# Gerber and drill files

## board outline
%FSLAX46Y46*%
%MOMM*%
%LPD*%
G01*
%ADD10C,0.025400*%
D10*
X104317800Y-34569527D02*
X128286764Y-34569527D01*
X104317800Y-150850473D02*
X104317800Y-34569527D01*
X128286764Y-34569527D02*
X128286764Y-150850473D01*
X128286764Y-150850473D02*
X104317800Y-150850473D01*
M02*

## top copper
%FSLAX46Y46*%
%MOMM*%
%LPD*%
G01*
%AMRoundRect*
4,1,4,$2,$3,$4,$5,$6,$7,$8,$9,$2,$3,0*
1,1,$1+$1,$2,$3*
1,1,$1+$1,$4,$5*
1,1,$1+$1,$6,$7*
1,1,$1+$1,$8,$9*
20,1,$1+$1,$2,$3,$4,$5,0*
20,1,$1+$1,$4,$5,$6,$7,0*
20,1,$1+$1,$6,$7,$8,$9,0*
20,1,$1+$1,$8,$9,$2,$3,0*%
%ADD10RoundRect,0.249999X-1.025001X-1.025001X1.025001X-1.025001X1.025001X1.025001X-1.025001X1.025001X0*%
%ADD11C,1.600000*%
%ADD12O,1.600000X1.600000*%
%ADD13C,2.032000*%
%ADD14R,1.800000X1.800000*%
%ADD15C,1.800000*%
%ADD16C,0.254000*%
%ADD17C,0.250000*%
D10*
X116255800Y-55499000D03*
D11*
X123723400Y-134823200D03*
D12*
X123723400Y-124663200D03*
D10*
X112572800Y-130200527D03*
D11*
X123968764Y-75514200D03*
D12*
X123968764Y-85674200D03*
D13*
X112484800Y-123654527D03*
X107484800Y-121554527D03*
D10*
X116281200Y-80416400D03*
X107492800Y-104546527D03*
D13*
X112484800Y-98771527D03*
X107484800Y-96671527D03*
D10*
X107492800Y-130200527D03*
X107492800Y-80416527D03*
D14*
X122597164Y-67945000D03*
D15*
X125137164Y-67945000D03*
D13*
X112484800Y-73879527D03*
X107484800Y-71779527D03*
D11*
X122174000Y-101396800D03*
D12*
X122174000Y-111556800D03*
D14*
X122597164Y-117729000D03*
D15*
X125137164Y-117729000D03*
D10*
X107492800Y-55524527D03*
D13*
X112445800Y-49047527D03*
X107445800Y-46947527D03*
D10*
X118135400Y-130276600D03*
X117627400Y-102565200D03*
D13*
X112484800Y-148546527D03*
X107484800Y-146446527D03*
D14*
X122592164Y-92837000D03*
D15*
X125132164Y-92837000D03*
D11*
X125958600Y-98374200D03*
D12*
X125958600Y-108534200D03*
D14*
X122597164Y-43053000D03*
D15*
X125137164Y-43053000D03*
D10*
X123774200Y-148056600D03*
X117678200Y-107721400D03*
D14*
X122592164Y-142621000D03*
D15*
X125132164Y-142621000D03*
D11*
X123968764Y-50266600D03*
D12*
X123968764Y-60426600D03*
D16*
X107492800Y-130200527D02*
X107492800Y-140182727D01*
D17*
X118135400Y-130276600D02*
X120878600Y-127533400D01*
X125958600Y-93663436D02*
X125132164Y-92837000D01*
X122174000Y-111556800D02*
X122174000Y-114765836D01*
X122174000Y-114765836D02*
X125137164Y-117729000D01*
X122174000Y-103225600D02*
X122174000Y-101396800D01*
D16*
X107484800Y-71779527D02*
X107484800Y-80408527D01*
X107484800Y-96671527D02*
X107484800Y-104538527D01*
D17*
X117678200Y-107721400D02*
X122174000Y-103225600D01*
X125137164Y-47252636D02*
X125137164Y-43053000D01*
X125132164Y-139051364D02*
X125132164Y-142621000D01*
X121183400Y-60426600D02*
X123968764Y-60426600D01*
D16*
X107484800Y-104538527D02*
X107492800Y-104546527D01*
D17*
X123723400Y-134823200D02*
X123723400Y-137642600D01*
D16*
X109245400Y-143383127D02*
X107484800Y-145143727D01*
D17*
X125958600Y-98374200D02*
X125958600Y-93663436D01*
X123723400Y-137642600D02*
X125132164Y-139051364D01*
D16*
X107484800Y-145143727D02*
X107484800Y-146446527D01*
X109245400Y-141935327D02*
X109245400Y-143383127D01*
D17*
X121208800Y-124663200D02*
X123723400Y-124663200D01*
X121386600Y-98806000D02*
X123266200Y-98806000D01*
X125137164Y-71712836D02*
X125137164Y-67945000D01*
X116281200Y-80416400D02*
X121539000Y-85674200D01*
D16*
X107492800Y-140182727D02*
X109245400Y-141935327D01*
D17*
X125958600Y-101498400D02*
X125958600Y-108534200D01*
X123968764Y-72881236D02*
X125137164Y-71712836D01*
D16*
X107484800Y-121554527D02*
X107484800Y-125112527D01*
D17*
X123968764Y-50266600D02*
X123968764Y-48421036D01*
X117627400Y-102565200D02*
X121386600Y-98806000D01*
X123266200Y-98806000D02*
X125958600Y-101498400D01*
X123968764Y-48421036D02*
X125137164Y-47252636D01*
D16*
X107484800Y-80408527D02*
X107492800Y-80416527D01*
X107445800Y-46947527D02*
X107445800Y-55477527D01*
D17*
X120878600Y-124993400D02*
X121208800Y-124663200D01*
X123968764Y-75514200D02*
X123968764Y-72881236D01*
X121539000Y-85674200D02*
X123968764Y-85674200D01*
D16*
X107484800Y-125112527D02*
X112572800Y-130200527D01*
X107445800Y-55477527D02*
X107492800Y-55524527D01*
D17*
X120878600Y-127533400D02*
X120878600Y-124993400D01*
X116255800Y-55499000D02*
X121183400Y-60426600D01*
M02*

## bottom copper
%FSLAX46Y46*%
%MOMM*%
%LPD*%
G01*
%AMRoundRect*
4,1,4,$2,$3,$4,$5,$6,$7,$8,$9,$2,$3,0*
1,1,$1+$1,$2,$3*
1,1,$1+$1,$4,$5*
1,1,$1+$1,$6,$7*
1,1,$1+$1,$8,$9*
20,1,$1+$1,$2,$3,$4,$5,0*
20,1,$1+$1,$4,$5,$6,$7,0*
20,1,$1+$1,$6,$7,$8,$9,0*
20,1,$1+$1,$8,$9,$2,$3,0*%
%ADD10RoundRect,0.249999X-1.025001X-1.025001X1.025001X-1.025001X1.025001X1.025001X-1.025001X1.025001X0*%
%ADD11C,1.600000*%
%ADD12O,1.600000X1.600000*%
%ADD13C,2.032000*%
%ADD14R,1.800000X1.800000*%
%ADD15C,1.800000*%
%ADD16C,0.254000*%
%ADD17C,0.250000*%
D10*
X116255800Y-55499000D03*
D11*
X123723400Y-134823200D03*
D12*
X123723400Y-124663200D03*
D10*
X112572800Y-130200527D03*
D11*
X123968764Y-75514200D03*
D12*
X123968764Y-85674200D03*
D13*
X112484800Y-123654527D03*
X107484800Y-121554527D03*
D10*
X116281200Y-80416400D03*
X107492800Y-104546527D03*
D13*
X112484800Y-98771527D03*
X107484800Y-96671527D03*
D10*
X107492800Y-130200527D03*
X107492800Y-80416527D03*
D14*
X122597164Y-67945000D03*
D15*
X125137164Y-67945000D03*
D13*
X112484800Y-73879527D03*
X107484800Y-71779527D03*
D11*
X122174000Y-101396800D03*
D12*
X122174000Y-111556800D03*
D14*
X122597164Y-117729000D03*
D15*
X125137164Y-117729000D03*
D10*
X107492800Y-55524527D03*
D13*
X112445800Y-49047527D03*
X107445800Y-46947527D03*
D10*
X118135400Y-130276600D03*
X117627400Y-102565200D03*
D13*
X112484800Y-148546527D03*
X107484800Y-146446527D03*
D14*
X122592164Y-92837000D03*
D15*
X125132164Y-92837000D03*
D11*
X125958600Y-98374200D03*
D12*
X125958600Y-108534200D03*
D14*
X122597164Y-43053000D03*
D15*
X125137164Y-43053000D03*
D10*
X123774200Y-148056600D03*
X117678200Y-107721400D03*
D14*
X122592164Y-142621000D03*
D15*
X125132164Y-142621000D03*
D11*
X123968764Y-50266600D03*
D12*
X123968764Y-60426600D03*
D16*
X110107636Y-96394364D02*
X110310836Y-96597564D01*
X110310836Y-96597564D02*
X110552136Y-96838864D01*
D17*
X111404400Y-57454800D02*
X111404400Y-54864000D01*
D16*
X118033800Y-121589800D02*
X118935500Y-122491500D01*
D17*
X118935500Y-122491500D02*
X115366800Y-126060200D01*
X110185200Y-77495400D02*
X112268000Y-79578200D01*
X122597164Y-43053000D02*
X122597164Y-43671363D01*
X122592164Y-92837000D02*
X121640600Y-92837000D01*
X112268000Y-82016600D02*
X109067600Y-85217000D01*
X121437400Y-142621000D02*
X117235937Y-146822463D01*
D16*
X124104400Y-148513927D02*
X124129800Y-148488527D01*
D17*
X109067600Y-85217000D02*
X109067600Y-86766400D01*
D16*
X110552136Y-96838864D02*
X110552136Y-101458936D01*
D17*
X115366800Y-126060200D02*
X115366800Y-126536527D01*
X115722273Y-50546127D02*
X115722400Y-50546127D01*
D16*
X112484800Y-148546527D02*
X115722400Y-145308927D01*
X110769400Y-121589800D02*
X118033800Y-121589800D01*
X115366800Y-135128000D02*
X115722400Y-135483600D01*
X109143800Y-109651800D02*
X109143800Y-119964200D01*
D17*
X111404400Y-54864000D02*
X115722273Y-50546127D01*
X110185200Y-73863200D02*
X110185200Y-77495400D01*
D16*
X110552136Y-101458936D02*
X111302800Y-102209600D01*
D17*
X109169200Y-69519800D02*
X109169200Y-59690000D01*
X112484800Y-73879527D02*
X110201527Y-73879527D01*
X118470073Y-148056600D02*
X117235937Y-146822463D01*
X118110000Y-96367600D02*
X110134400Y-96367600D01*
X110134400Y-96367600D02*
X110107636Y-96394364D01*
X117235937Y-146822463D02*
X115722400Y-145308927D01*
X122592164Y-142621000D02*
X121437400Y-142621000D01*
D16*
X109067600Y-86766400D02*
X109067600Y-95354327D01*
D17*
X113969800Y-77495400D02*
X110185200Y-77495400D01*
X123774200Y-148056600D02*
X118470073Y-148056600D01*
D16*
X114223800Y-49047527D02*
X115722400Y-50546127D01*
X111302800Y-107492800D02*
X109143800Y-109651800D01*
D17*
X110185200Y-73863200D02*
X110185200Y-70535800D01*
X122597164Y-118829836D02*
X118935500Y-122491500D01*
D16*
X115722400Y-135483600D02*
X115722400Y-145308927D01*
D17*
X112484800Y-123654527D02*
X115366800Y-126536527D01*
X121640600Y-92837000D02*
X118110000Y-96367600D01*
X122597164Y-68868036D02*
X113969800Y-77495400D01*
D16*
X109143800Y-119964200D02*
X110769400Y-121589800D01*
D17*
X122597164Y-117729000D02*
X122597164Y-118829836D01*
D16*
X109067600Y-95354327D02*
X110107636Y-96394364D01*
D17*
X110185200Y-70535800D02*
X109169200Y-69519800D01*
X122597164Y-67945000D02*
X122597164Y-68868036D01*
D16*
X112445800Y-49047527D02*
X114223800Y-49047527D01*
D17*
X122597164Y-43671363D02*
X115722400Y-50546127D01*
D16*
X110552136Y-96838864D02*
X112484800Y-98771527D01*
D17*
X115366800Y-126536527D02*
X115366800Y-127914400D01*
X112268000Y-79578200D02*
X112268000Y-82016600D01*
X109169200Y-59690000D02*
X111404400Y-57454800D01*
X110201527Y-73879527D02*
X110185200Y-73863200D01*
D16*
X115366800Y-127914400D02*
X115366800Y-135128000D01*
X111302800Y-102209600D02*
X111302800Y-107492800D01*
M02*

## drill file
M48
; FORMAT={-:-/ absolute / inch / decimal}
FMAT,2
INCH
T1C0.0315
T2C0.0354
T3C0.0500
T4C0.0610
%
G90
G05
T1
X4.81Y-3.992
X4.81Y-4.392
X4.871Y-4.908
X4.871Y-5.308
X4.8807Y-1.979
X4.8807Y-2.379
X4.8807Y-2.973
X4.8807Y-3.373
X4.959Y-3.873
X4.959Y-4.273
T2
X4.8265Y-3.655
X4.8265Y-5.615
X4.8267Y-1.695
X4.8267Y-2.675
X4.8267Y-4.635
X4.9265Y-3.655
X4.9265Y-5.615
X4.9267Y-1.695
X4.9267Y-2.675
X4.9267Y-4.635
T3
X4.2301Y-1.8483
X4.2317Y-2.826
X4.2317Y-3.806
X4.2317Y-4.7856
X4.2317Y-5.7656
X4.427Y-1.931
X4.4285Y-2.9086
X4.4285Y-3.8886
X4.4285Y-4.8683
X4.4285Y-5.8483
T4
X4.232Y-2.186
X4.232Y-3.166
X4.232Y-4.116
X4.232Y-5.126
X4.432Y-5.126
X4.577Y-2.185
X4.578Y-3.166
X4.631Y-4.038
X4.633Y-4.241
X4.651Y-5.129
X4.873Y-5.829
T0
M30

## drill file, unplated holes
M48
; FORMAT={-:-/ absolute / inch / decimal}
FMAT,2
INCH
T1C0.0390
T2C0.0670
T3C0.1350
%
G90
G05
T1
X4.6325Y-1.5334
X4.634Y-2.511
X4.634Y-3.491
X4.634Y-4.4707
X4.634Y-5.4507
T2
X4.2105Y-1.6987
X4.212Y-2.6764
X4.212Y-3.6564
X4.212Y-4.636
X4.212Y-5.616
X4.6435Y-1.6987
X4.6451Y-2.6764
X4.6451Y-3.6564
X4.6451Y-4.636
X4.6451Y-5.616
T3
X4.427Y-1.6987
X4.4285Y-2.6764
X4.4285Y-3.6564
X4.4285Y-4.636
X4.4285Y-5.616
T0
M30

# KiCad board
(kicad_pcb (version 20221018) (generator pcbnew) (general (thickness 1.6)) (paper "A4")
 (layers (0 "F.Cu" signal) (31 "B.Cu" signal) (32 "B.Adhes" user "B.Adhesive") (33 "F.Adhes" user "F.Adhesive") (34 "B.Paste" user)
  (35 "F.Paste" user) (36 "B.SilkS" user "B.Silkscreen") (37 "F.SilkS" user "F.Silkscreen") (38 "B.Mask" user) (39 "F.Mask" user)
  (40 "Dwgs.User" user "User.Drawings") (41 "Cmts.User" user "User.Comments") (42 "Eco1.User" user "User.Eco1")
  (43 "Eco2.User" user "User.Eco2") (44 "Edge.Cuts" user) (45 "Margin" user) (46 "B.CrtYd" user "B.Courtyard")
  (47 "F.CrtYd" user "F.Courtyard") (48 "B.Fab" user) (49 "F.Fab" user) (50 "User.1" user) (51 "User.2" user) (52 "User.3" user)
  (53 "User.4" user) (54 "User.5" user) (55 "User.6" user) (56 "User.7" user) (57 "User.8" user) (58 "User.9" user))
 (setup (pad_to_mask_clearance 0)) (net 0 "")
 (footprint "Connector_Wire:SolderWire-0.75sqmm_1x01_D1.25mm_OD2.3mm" (layer "F.Cu") (at 116.2558 55.499)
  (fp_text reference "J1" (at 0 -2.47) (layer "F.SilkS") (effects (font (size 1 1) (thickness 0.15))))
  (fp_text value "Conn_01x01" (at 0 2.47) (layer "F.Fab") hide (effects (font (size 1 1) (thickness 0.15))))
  (pad "1" thru_hole roundrect (at 0 0) (size 2.55 2.55) (drill 1.55) (layers "*.Cu" "*.Mask") (roundrect_rratio 0.09803882353)))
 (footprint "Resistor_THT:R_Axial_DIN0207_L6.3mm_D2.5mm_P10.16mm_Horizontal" (layer "F.Cu") (at 123.7234 134.8232 90)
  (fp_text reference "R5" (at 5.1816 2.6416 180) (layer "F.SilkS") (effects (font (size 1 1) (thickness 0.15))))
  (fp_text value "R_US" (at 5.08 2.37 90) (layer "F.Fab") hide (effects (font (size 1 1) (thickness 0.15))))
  (pad "1" thru_hole circle (at 0 0 90) (size 1.6 1.6) (drill 0.8) (layers "*.Cu" "*.Mask"))
  (pad "2" thru_hole oval (at 10.16 0 90) (size 1.6 1.6) (drill 0.8) (layers "*.Cu" "*.Mask")))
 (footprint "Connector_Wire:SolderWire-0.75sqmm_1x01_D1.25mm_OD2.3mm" (layer "F.Cu") (at 112.5728 130.200527)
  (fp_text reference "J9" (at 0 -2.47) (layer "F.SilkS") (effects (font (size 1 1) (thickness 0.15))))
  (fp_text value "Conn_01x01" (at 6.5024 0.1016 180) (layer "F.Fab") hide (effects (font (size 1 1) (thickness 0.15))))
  (pad "1" thru_hole roundrect (at 0 0) (size 2.55 2.55) (drill 1.55) (layers "*.Cu" "*.Mask") (roundrect_rratio 0.09803882353)))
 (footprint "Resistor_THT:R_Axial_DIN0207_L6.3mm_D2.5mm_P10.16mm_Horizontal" (layer "F.Cu") (at 123.968764 75.5142 -90)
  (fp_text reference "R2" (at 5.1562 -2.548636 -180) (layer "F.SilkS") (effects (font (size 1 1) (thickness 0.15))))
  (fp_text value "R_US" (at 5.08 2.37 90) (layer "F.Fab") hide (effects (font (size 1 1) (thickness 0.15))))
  (pad "1" thru_hole circle (at 0 0 270) (size 1.6 1.6) (drill 0.8) (layers "*.Cu" "*.Mask"))
  (pad "2" thru_hole oval (at 10.16 0 270) (size 1.6 1.6) (drill 0.8) (layers "*.Cu" "*.Mask")))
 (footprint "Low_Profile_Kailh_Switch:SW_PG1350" (layer "F.Cu") (at 112.4848 117.754527)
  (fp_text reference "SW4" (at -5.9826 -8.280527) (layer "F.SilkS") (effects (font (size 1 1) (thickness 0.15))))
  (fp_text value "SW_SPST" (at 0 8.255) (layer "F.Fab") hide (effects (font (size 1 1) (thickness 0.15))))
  (pad "" np_thru_hole circle (at -5.5 0) (size 1.7018 1.7018) (drill 1.7018) (layers "F&B.Cu" "*.Mask"))
  (pad "" np_thru_hole circle (at 0 0) (size 3.429 3.429) (drill 3.429) (layers "F&B.Cu" "*.Mask"))
  (pad "" np_thru_hole circle (at 5.22 -4.2) (size 0.9906 0.9906) (drill 0.9906) (layers "F&B.Cu" "*.Mask"))
  (pad "" np_thru_hole circle (at 5.5 0) (size 1.7018 1.7018) (drill 1.7018) (layers "F&B.Cu" "*.Mask"))
  (pad "1" thru_hole circle (at 0 5.9) (size 2.032 2.032) (drill 1.27) (layers "*.Cu" "*.Mask"))
  (pad "2" thru_hole circle (at -5 3.8) (size 2.032 2.032) (drill 1.27) (layers "*.Cu" "*.Mask")))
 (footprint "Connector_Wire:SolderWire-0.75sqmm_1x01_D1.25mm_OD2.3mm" (layer "F.Cu") (at 116.2812 80.4164)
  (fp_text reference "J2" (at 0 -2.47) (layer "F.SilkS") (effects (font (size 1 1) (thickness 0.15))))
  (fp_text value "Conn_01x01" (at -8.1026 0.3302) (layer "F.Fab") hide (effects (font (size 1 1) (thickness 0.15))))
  (pad "1" thru_hole roundrect (at 0 0) (size 2.55 2.55) (drill 1.55) (layers "*.Cu" "*.Mask") (roundrect_rratio 0.09803882353)))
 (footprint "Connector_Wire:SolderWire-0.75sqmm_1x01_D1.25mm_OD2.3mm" (layer "F.Cu") (at 107.4928 104.546527)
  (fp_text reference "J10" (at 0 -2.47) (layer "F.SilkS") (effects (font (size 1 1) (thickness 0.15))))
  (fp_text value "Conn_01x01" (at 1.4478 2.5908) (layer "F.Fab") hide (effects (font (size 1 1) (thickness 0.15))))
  (pad "1" thru_hole roundrect (at 0 0) (size 2.55 2.55) (drill 1.55) (layers "*.Cu" "*.Mask") (roundrect_rratio 0.09803882353)))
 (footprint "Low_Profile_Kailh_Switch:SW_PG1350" (layer "F.Cu") (at 112.4848 92.871527)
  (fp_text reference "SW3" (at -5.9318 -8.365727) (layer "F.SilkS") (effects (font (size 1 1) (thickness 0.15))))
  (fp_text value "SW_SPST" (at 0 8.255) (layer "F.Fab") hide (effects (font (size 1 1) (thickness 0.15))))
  (pad "" np_thru_hole circle (at -5.5 0) (size 1.7018 1.7018) (drill 1.7018) (layers "F&B.Cu" "*.Mask"))
  (pad "" np_thru_hole circle (at 0 0) (size 3.429 3.429) (drill 3.429) (layers "F&B.Cu" "*.Mask"))
  (pad "" np_thru_hole circle (at 5.22 -4.2) (size 0.9906 0.9906) (drill 0.9906) (layers "F&B.Cu" "*.Mask"))
  (pad "" np_thru_hole circle (at 5.5 0) (size 1.7018 1.7018) (drill 1.7018) (layers "F&B.Cu" "*.Mask"))
  (pad "1" thru_hole circle (at 0 5.9) (size 2.032 2.032) (drill 1.27) (layers "*.Cu" "*.Mask"))
  (pad "2" thru_hole circle (at -5 3.8) (size 2.032 2.032) (drill 1.27) (layers "*.Cu" "*.Mask")))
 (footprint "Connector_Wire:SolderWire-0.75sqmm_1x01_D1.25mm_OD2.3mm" (layer "F.Cu") (at 107.4928 130.200527)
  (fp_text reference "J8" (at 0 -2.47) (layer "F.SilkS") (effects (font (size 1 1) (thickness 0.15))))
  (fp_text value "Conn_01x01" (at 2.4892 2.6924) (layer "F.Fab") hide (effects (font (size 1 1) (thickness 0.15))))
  (pad "1" thru_hole roundrect (at 0 0) (size 2.55 2.55) (drill 1.55) (layers "*.Cu" "*.Mask") (roundrect_rratio 0.09803882353)))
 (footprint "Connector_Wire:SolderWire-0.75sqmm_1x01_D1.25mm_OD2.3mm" (layer "F.Cu") (at 107.4928 80.416527)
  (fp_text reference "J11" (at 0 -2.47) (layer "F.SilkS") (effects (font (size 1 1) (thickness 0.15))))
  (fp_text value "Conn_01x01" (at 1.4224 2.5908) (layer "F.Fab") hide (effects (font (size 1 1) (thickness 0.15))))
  (pad "1" thru_hole roundrect (at 0 0) (size 2.55 2.55) (drill 1.55) (layers "*.Cu" "*.Mask") (roundrect_rratio 0.09803882353)))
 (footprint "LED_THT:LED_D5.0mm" (layer "F.Cu") (at 122.597164 67.945)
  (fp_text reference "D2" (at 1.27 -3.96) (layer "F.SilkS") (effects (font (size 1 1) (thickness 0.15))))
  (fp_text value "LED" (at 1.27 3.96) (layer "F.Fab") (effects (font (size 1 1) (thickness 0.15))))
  (pad "1" thru_hole rect (at 0 0) (size 1.8 1.8) (drill 0.9) (layers "*.Cu" "*.Mask"))
  (pad "2" thru_hole circle (at 2.54 0) (size 1.8 1.8) (drill 0.9) (layers "*.Cu" "*.Mask")))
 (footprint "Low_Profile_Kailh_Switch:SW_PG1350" (layer "F.Cu") (at 112.4848 67.979527)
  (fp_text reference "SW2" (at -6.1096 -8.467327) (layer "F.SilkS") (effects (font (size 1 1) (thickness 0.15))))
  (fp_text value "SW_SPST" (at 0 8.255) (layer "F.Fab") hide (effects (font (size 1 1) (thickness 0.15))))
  (pad "" np_thru_hole circle (at -5.5 0) (size 1.7018 1.7018) (drill 1.7018) (layers "F&B.Cu" "*.Mask"))
  (pad "" np_thru_hole circle (at 0 0) (size 3.429 3.429) (drill 3.429) (layers "F&B.Cu" "*.Mask"))
  (pad "" np_thru_hole circle (at 5.22 -4.2) (size 0.9906 0.9906) (drill 0.9906) (layers "F&B.Cu" "*.Mask"))
  (pad "" np_thru_hole circle (at 5.5 0) (size 1.7018 1.7018) (drill 1.7018) (layers "F&B.Cu" "*.Mask"))
  (pad "1" thru_hole circle (at 0 5.9) (size 2.032 2.032) (drill 1.27) (layers "*.Cu" "*.Mask"))
  (pad "2" thru_hole circle (at -5 3.8) (size 2.032 2.032) (drill 1.27) (layers "*.Cu" "*.Mask")))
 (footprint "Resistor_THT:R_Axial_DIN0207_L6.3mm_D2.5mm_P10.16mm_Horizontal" (layer "F.Cu") (at 122.174 101.3968 -90)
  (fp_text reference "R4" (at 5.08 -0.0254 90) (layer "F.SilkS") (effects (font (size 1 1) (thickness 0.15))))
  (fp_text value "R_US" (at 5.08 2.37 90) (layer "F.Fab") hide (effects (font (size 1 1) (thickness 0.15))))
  (pad "1" thru_hole circle (at 0 0 270) (size 1.6 1.6) (drill 0.8) (layers "*.Cu" "*.Mask"))
  (pad "2" thru_hole oval (at 10.16 0 270) (size 1.6 1.6) (drill 0.8) (layers "*.Cu" "*.Mask")))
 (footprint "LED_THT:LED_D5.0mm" (layer "F.Cu") (at 122.597164 117.729)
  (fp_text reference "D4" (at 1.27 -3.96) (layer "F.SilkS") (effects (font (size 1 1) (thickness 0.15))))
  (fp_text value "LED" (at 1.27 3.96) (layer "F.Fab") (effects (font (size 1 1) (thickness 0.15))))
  (pad "1" thru_hole rect (at 0 0) (size 1.8 1.8) (drill 0.9) (layers "*.Cu" "*.Mask"))
  (pad "2" thru_hole circle (at 2.54 0) (size 1.8 1.8) (drill 0.9) (layers "*.Cu" "*.Mask")))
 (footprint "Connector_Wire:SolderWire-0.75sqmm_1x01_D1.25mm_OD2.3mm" (layer "F.Cu") (at 107.4928 55.524527)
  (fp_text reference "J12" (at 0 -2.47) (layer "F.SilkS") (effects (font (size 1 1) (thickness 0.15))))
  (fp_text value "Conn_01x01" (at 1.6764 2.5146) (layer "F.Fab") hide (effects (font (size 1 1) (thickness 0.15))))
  (pad "1" thru_hole roundrect (at 0 0) (size 2.55 2.55) (drill 1.55) (layers "*.Cu" "*.Mask") (roundrect_rratio 0.09803882353)))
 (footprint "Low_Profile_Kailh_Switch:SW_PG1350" (layer "F.Cu") (at 112.4458 43.147527)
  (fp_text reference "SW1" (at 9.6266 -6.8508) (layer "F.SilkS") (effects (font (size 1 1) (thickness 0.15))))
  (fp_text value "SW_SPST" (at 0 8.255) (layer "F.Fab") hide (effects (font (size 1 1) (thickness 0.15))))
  (pad "" np_thru_hole circle (at -5.5 0) (size 1.7018 1.7018) (drill 1.7018) (layers "F&B.Cu" "*.Mask"))
  (pad "" np_thru_hole circle (at 0 0) (size 3.429 3.429) (drill 3.429) (layers "F&B.Cu" "*.Mask"))
  (pad "" np_thru_hole circle (at 5.22 -4.2) (size 0.9906 0.9906) (drill 0.9906) (layers "F&B.Cu" "*.Mask"))
  (pad "" np_thru_hole circle (at 5.5 0) (size 1.7018 1.7018) (drill 1.7018) (layers "F&B.Cu" "*.Mask"))
  (pad "1" thru_hole circle (at 0 5.9) (size 2.032 2.032) (drill 1.27) (layers "*.Cu" "*.Mask"))
  (pad "2" thru_hole circle (at -5 3.8) (size 2.032 2.032) (drill 1.27) (layers "*.Cu" "*.Mask")))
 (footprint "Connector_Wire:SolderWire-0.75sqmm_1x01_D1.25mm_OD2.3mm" (layer "F.Cu") (at 118.1354 130.2766)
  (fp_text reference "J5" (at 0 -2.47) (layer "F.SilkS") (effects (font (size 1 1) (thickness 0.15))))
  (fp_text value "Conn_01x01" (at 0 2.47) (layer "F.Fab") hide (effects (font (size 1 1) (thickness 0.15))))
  (pad "1" thru_hole roundrect (at 0 0) (size 2.55 2.55) (drill 1.55) (layers "*.Cu" "*.Mask") (roundrect_rratio 0.09803882353)))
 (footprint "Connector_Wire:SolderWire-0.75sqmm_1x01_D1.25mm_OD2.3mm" (layer "F.Cu") (at 117.6274 102.5652)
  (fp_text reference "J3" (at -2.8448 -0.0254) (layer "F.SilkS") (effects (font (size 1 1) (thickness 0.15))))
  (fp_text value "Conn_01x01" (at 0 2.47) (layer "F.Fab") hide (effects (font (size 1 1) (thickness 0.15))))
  (pad "1" thru_hole roundrect (at 0 0) (size 2.55 2.55) (drill 1.55) (layers "*.Cu" "*.Mask") (roundrect_rratio 0.09803882353)))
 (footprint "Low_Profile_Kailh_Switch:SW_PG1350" (layer "F.Cu") (at 112.4848 142.646527)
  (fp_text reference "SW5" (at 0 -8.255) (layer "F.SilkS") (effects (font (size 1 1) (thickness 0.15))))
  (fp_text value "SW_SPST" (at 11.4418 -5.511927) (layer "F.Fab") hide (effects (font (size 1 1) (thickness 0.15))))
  (pad "" np_thru_hole circle (at -5.5 0) (size 1.7018 1.7018) (drill 1.7018) (layers "F&B.Cu" "*.Mask"))
  (pad "" np_thru_hole circle (at 0 0) (size 3.429 3.429) (drill 3.429) (layers "F&B.Cu" "*.Mask"))
  (pad "" np_thru_hole circle (at 5.22 -4.2) (size 0.9906 0.9906) (drill 0.9906) (layers "F&B.Cu" "*.Mask"))
  (pad "" np_thru_hole circle (at 5.5 0) (size 1.7018 1.7018) (drill 1.7018) (layers "F&B.Cu" "*.Mask"))
  (pad "1" thru_hole circle (at 0 5.9) (size 2.032 2.032) (drill 1.27) (layers "*.Cu" "*.Mask"))
  (pad "2" thru_hole circle (at -5 3.8) (size 2.032 2.032) (drill 1.27) (layers "*.Cu" "*.Mask")))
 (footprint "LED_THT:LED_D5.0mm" (layer "F.Cu") (at 122.592164 92.837)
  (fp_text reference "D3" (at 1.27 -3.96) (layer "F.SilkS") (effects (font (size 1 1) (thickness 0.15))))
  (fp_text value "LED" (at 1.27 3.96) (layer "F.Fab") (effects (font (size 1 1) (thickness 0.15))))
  (pad "1" thru_hole rect (at 0 0) (size 1.8 1.8) (drill 0.9) (layers "*.Cu" "*.Mask"))
  (pad "2" thru_hole circle (at 2.54 0) (size 1.8 1.8) (drill 0.9) (layers "*.Cu" "*.Mask")))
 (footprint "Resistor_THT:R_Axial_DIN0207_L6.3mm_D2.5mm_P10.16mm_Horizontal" (layer "F.Cu") (at 125.9586 98.3742 -90)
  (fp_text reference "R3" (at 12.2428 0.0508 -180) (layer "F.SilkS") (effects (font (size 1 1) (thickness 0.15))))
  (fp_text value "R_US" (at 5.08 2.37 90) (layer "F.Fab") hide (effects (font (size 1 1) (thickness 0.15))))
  (pad "1" thru_hole circle (at 0 0 270) (size 1.6 1.6) (drill 0.8) (layers "*.Cu" "*.Mask"))
  (pad "2" thru_hole oval (at 10.16 0 270) (size 1.6 1.6) (drill 0.8) (layers "*.Cu" "*.Mask")))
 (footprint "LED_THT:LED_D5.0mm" (layer "F.Cu") (at 122.597164 43.053)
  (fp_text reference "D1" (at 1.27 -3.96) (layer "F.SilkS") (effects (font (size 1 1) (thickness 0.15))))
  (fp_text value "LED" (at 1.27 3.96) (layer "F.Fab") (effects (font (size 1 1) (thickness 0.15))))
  (pad "1" thru_hole rect (at 0 0) (size 1.8 1.8) (drill 0.9) (layers "*.Cu" "*.Mask"))
  (pad "2" thru_hole circle (at 2.54 0) (size 1.8 1.8) (drill 0.9) (layers "*.Cu" "*.Mask")))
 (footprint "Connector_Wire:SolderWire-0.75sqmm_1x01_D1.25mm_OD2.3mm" (layer "F.Cu") (at 123.7742 148.0566)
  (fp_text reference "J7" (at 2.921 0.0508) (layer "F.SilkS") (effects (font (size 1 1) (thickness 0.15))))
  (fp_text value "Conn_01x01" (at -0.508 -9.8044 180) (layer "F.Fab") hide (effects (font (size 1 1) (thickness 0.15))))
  (pad "1" thru_hole roundrect (at 0 0) (size 2.55 2.55) (drill 1.55) (layers "*.Cu" "*.Mask") (roundrect_rratio 0.09803882353)))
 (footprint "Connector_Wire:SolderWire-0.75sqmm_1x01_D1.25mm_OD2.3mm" (layer "F.Cu") (at 117.6782 107.7214)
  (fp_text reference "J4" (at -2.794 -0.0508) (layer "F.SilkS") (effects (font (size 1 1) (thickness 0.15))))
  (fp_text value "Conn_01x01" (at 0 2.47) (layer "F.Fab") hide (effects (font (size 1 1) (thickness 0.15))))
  (pad "1" thru_hole roundrect (at 0 0) (size 2.55 2.55) (drill 1.55) (layers "*.Cu" "*.Mask") (roundrect_rratio 0.09803882353)))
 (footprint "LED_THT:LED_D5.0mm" (layer "F.Cu") (at 122.592164 142.621)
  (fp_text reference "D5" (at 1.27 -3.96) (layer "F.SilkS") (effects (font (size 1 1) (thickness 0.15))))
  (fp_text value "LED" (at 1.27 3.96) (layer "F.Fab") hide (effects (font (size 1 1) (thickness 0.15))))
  (pad "1" thru_hole rect (at 0 0) (size 1.8 1.8) (drill 0.9) (layers "*.Cu" "*.Mask"))
  (pad "2" thru_hole circle (at 2.54 0) (size 1.8 1.8) (drill 0.9) (layers "*.Cu" "*.Mask")))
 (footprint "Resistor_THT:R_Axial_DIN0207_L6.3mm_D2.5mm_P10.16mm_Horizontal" (layer "F.Cu") (at 123.968764 50.2666 -90)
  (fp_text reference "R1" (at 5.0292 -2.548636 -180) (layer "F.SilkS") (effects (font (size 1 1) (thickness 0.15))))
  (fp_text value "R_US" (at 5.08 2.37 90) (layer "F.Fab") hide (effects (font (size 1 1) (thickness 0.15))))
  (pad "1" thru_hole circle (at 0 0 270) (size 1.6 1.6) (drill 0.8) (layers "*.Cu" "*.Mask"))
  (pad "2" thru_hole oval (at 10.16 0 270) (size 1.6 1.6) (drill 0.8) (layers "*.Cu" "*.Mask")))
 (gr_line (start 104.3178 34.569527) (end 128.286764 34.569527) (stroke (width 0.0254) (type default)) (layer "Edge.Cuts"))
 (gr_line (start 104.3178 150.850473) (end 104.3178 34.569527) (stroke (width 0.0254) (type default)) (layer "Edge.Cuts"))
 (gr_line (start 128.286764 34.569527) (end 128.286764 150.850473) (stroke (width 0.0254) (type default)) (layer "Edge.Cuts"))
 (gr_line (start 128.286764 150.850473) (end 104.3178 150.850473) (stroke (width 0.0254) (type default)) (layer "Edge.Cuts"))
 (segment (start 107.4928 130.200527) (end 107.4928 140.182727) (width 0.254) (layer "F.Cu") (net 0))
 (segment (start 118.1354 130.2766) (end 120.8786 127.5334) (width 0.25) (layer "F.Cu") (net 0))
 (segment (start 125.9586 93.663436) (end 125.132164 92.837) (width 0.25) (layer "F.Cu") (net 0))
 (segment (start 122.174 111.5568) (end 122.174 114.765836) (width 0.25) (layer "F.Cu") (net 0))
 (segment (start 122.174 114.765836) (end 125.137164 117.729) (width 0.25) (layer "F.Cu") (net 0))
 (segment (start 122.174 103.2256) (end 122.174 101.3968) (width 0.25) (layer "F.Cu") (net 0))
 (segment (start 107.4848 71.779527) (end 107.4848 80.408527) (width 0.254) (layer "F.Cu") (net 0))
 (segment (start 107.4848 96.671527) (end 107.4848 104.538527) (width 0.254) (layer "F.Cu") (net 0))
 (segment (start 117.6782 107.7214) (end 122.174 103.2256) (width 0.25) (layer "F.Cu") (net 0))
 (segment (start 125.137164 47.252636) (end 125.137164 43.053) (width 0.25) (layer "F.Cu") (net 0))
 (segment (start 125.132164 139.051364) (end 125.132164 142.621) (width 0.25) (layer "F.Cu") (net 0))
 (segment (start 121.1834 60.4266) (end 123.968764 60.4266) (width 0.25) (layer "F.Cu") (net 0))
 (segment (start 107.4848 104.538527) (end 107.4928 104.546527) (width 0.254) (layer "F.Cu") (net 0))
 (segment (start 123.7234 134.8232) (end 123.7234 137.6426) (width 0.25) (layer "F.Cu") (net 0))
 (segment (start 109.2454 143.383127) (end 107.4848 145.143727) (width 0.254) (layer "F.Cu") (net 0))
 (segment (start 125.9586 98.3742) (end 125.9586 93.663436) (width 0.25) (layer "F.Cu") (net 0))
 (segment (start 123.7234 137.6426) (end 125.132164 139.051364) (width 0.25) (layer "F.Cu") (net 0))
 (segment (start 107.4848 145.143727) (end 107.4848 146.446527) (width 0.254) (layer "F.Cu") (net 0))
 (segment (start 109.2454 141.935327) (end 109.2454 143.383127) (width 0.254) (layer "F.Cu") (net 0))
 (segment (start 121.2088 124.6632) (end 123.7234 124.6632) (width 0.25) (layer "F.Cu") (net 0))
 (segment (start 121.3866 98.806) (end 123.2662 98.806) (width 0.25) (layer "F.Cu") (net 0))
 (segment (start 125.137164 71.712836) (end 125.137164 67.945) (width 0.25) (layer "F.Cu") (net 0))
 (segment (start 116.2812 80.4164) (end 121.539 85.6742) (width 0.25) (layer "F.Cu") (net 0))
 (segment (start 107.4928 140.182727) (end 109.2454 141.935327) (width 0.254) (layer "F.Cu") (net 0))
 (segment (start 125.9586 101.4984) (end 125.9586 108.5342) (width 0.25) (layer "F.Cu") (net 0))
 (segment (start 123.968764 72.881236) (end 125.137164 71.712836) (width 0.25) (layer "F.Cu") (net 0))
 (segment (start 107.4848 121.554527) (end 107.4848 125.112527) (width 0.254) (layer "F.Cu") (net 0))
 (segment (start 123.968764 50.2666) (end 123.968764 48.421036) (width 0.25) (layer "F.Cu") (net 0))
 (segment (start 117.6274 102.5652) (end 121.3866 98.806) (width 0.25) (layer "F.Cu") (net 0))
 (segment (start 123.2662 98.806) (end 125.9586 101.4984) (width 0.25) (layer "F.Cu") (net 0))
 (segment (start 123.968764 48.421036) (end 125.137164 47.252636) (width 0.25) (layer "F.Cu") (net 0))
 (segment (start 107.4848 80.408527) (end 107.4928 80.416527) (width 0.254) (layer "F.Cu") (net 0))
 (segment (start 107.4458 46.947527) (end 107.4458 55.477527) (width 0.254) (layer "F.Cu") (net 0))
 (segment (start 120.8786 124.9934) (end 121.2088 124.6632) (width 0.25) (layer "F.Cu") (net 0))
 (segment (start 123.968764 75.5142) (end 123.968764 72.881236) (width 0.25) (layer "F.Cu") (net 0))
 (segment (start 121.539 85.6742) (end 123.968764 85.6742) (width 0.25) (layer "F.Cu") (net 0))
 (segment (start 107.4848 125.112527) (end 112.5728 130.200527) (width 0.254) (layer "F.Cu") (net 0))
 (segment (start 107.4458 55.477527) (end 107.4928 55.524527) (width 0.254) (layer "F.Cu") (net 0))
 (segment (start 120.8786 127.5334) (end 120.8786 124.9934) (width 0.25) (layer "F.Cu") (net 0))
 (segment (start 116.2558 55.499) (end 121.1834 60.4266) (width 0.25) (layer "F.Cu") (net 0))
 (segment (start 110.107636 96.394364) (end 110.310836 96.597564) (width 0.254) (layer "B.Cu") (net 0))
 (segment (start 110.310836 96.597564) (end 110.552136 96.838864) (width 0.254) (layer "B.Cu") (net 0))
 (segment (start 111.4044 57.4548) (end 111.4044 54.864) (width 0.25) (layer "B.Cu") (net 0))
 (segment (start 118.0338 121.5898) (end 118.9355 122.4915) (width 0.254) (layer "B.Cu") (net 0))
 (segment (start 118.9355 122.4915) (end 115.3668 126.0602) (width 0.25) (layer "B.Cu") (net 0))
 (segment (start 110.1852 77.4954) (end 112.268 79.5782) (width 0.25) (layer "B.Cu") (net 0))
 (segment (start 122.597164 43.053) (end 122.597164 43.671363) (width 0.25) (layer "B.Cu") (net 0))
 (segment (start 122.592164 92.837) (end 121.6406 92.837) (width 0.25) (layer "B.Cu") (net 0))
 (segment (start 112.268 82.0166) (end 109.0676 85.217) (width 0.25) (layer "B.Cu") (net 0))
 (segment (start 121.4374 142.621) (end 117.235937 146.822463) (width 0.25) (layer "B.Cu") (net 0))
 (segment (start 124.1044 148.513927) (end 124.1298 148.488527) (width 0.254) (layer "B.Cu") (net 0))
 (segment (start 109.0676 85.217) (end 109.0676 86.7664) (width 0.25) (layer "B.Cu") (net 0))
 (segment (start 110.552136 96.838864) (end 110.552136 101.458936) (width 0.254) (layer "B.Cu") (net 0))
 (segment (start 115.3668 126.0602) (end 115.3668 126.536527) (width 0.25) (layer "B.Cu") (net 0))
 (segment (start 115.722273 50.546127) (end 115.7224 50.546127) (width 0.25) (layer "B.Cu") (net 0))
 (segment (start 112.4848 148.546527) (end 115.7224 145.308927) (width 0.254) (layer "B.Cu") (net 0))
 (segment (start 110.7694 121.5898) (end 118.0338 121.5898) (width 0.254) (layer "B.Cu") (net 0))
 (segment (start 115.3668 135.128) (end 115.7224 135.4836) (width 0.254) (layer "B.Cu") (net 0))
 (segment (start 109.1438 109.6518) (end 109.1438 119.9642) (width 0.254) (layer "B.Cu") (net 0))
 (segment (start 111.4044 54.864) (end 115.722273 50.546127) (width 0.25) (layer "B.Cu") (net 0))
 (segment (start 110.1852 73.8632) (end 110.1852 77.4954) (width 0.25) (layer "B.Cu") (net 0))
 (segment (start 110.552136 101.458936) (end 111.3028 102.2096) (width 0.254) (layer "B.Cu") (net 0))
 (segment (start 109.1692 69.5198) (end 109.1692 59.69) (width 0.25) (layer "B.Cu") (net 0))
 (segment (start 112.4848 73.879527) (end 110.201527 73.879527) (width 0.25) (layer "B.Cu") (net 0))
 (segment (start 118.470073 148.0566) (end 117.235937 146.822463) (width 0.25) (layer "B.Cu") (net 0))
 (segment (start 118.11 96.3676) (end 110.1344 96.3676) (width 0.25) (layer "B.Cu") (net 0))
 (segment (start 110.1344 96.3676) (end 110.107636 96.394364) (width 0.25) (layer "B.Cu") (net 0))
 (segment (start 117.235937 146.822463) (end 115.7224 145.308927) (width 0.25) (layer "B.Cu") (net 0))
 (segment (start 122.592164 142.621) (end 121.4374 142.621) (width 0.25) (layer "B.Cu") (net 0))
 (segment (start 109.0676 86.7664) (end 109.0676 95.354327) (width 0.254) (layer "B.Cu") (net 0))
 (segment (start 113.9698 77.4954) (end 110.1852 77.4954) (width 0.25) (layer "B.Cu") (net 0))
 (segment (start 123.7742 148.0566) (end 118.470073 148.0566) (width 0.25) (layer "B.Cu") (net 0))
 (segment (start 114.2238 49.047527) (end 115.7224 50.546127) (width 0.254) (layer "B.Cu") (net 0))
 (segment (start 111.3028 107.4928) (end 109.1438 109.6518) (width 0.254) (layer "B.Cu") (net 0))
 (segment (start 110.1852 73.8632) (end 110.1852 70.5358) (width 0.25) (layer "B.Cu") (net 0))
 (segment (start 122.597164 118.829836) (end 118.9355 122.4915) (width 0.25) (layer "B.Cu") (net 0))
 (segment (start 115.7224 135.4836) (end 115.7224 145.308927) (width 0.254) (layer "B.Cu") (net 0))
 (segment (start 112.4848 123.654527) (end 115.3668 126.536527) (width 0.25) (layer "B.Cu") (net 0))
 (segment (start 121.6406 92.837) (end 118.11 96.3676) (width 0.25) (layer "B.Cu") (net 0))
 (segment (start 122.597164 68.868036) (end 113.9698 77.4954) (width 0.25) (layer "B.Cu") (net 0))
 (segment (start 109.1438 119.9642) (end 110.7694 121.5898) (width 0.254) (layer "B.Cu") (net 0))
 (segment (start 122.597164 117.729) (end 122.597164 118.829836) (width 0.25) (layer "B.Cu") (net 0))
 (segment (start 109.0676 95.354327) (end 110.107636 96.394364) (width 0.254) (layer "B.Cu") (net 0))
 (segment (start 110.1852 70.5358) (end 109.1692 69.5198) (width 0.25) (layer "B.Cu") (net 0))
 (segment (start 122.597164 67.945) (end 122.597164 68.868036) (width 0.25) (layer "B.Cu") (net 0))
 (segment (start 112.4458 49.047527) (end 114.2238 49.047527) (width 0.254) (layer "B.Cu") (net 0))
 (segment (start 122.597164 43.671363) (end 115.7224 50.546127) (width 0.25) (layer "B.Cu") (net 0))
 (segment (start 110.552136 96.838864) (end 112.4848 98.771527) (width 0.254) (layer "B.Cu") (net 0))
 (segment (start 115.3668 126.536527) (end 115.3668 127.9144) (width 0.25) (layer "B.Cu") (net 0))
 (segment (start 112.268 79.5782) (end 112.268 82.0166) (width 0.25) (layer "B.Cu") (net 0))
 (segment (start 109.1692 59.69) (end 111.4044 57.4548) (width 0.25) (layer "B.Cu") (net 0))
 (segment (start 110.201527 73.879527) (end 110.1852 73.8632) (width 0.25) (layer "B.Cu") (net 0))
 (segment (start 115.3668 127.9144) (end 115.3668 135.128) (width 0.254) (layer "B.Cu") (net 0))
 (segment (start 111.3028 102.2096) (end 111.3028 107.4928) (width 0.254) (layer "B.Cu") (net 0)))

